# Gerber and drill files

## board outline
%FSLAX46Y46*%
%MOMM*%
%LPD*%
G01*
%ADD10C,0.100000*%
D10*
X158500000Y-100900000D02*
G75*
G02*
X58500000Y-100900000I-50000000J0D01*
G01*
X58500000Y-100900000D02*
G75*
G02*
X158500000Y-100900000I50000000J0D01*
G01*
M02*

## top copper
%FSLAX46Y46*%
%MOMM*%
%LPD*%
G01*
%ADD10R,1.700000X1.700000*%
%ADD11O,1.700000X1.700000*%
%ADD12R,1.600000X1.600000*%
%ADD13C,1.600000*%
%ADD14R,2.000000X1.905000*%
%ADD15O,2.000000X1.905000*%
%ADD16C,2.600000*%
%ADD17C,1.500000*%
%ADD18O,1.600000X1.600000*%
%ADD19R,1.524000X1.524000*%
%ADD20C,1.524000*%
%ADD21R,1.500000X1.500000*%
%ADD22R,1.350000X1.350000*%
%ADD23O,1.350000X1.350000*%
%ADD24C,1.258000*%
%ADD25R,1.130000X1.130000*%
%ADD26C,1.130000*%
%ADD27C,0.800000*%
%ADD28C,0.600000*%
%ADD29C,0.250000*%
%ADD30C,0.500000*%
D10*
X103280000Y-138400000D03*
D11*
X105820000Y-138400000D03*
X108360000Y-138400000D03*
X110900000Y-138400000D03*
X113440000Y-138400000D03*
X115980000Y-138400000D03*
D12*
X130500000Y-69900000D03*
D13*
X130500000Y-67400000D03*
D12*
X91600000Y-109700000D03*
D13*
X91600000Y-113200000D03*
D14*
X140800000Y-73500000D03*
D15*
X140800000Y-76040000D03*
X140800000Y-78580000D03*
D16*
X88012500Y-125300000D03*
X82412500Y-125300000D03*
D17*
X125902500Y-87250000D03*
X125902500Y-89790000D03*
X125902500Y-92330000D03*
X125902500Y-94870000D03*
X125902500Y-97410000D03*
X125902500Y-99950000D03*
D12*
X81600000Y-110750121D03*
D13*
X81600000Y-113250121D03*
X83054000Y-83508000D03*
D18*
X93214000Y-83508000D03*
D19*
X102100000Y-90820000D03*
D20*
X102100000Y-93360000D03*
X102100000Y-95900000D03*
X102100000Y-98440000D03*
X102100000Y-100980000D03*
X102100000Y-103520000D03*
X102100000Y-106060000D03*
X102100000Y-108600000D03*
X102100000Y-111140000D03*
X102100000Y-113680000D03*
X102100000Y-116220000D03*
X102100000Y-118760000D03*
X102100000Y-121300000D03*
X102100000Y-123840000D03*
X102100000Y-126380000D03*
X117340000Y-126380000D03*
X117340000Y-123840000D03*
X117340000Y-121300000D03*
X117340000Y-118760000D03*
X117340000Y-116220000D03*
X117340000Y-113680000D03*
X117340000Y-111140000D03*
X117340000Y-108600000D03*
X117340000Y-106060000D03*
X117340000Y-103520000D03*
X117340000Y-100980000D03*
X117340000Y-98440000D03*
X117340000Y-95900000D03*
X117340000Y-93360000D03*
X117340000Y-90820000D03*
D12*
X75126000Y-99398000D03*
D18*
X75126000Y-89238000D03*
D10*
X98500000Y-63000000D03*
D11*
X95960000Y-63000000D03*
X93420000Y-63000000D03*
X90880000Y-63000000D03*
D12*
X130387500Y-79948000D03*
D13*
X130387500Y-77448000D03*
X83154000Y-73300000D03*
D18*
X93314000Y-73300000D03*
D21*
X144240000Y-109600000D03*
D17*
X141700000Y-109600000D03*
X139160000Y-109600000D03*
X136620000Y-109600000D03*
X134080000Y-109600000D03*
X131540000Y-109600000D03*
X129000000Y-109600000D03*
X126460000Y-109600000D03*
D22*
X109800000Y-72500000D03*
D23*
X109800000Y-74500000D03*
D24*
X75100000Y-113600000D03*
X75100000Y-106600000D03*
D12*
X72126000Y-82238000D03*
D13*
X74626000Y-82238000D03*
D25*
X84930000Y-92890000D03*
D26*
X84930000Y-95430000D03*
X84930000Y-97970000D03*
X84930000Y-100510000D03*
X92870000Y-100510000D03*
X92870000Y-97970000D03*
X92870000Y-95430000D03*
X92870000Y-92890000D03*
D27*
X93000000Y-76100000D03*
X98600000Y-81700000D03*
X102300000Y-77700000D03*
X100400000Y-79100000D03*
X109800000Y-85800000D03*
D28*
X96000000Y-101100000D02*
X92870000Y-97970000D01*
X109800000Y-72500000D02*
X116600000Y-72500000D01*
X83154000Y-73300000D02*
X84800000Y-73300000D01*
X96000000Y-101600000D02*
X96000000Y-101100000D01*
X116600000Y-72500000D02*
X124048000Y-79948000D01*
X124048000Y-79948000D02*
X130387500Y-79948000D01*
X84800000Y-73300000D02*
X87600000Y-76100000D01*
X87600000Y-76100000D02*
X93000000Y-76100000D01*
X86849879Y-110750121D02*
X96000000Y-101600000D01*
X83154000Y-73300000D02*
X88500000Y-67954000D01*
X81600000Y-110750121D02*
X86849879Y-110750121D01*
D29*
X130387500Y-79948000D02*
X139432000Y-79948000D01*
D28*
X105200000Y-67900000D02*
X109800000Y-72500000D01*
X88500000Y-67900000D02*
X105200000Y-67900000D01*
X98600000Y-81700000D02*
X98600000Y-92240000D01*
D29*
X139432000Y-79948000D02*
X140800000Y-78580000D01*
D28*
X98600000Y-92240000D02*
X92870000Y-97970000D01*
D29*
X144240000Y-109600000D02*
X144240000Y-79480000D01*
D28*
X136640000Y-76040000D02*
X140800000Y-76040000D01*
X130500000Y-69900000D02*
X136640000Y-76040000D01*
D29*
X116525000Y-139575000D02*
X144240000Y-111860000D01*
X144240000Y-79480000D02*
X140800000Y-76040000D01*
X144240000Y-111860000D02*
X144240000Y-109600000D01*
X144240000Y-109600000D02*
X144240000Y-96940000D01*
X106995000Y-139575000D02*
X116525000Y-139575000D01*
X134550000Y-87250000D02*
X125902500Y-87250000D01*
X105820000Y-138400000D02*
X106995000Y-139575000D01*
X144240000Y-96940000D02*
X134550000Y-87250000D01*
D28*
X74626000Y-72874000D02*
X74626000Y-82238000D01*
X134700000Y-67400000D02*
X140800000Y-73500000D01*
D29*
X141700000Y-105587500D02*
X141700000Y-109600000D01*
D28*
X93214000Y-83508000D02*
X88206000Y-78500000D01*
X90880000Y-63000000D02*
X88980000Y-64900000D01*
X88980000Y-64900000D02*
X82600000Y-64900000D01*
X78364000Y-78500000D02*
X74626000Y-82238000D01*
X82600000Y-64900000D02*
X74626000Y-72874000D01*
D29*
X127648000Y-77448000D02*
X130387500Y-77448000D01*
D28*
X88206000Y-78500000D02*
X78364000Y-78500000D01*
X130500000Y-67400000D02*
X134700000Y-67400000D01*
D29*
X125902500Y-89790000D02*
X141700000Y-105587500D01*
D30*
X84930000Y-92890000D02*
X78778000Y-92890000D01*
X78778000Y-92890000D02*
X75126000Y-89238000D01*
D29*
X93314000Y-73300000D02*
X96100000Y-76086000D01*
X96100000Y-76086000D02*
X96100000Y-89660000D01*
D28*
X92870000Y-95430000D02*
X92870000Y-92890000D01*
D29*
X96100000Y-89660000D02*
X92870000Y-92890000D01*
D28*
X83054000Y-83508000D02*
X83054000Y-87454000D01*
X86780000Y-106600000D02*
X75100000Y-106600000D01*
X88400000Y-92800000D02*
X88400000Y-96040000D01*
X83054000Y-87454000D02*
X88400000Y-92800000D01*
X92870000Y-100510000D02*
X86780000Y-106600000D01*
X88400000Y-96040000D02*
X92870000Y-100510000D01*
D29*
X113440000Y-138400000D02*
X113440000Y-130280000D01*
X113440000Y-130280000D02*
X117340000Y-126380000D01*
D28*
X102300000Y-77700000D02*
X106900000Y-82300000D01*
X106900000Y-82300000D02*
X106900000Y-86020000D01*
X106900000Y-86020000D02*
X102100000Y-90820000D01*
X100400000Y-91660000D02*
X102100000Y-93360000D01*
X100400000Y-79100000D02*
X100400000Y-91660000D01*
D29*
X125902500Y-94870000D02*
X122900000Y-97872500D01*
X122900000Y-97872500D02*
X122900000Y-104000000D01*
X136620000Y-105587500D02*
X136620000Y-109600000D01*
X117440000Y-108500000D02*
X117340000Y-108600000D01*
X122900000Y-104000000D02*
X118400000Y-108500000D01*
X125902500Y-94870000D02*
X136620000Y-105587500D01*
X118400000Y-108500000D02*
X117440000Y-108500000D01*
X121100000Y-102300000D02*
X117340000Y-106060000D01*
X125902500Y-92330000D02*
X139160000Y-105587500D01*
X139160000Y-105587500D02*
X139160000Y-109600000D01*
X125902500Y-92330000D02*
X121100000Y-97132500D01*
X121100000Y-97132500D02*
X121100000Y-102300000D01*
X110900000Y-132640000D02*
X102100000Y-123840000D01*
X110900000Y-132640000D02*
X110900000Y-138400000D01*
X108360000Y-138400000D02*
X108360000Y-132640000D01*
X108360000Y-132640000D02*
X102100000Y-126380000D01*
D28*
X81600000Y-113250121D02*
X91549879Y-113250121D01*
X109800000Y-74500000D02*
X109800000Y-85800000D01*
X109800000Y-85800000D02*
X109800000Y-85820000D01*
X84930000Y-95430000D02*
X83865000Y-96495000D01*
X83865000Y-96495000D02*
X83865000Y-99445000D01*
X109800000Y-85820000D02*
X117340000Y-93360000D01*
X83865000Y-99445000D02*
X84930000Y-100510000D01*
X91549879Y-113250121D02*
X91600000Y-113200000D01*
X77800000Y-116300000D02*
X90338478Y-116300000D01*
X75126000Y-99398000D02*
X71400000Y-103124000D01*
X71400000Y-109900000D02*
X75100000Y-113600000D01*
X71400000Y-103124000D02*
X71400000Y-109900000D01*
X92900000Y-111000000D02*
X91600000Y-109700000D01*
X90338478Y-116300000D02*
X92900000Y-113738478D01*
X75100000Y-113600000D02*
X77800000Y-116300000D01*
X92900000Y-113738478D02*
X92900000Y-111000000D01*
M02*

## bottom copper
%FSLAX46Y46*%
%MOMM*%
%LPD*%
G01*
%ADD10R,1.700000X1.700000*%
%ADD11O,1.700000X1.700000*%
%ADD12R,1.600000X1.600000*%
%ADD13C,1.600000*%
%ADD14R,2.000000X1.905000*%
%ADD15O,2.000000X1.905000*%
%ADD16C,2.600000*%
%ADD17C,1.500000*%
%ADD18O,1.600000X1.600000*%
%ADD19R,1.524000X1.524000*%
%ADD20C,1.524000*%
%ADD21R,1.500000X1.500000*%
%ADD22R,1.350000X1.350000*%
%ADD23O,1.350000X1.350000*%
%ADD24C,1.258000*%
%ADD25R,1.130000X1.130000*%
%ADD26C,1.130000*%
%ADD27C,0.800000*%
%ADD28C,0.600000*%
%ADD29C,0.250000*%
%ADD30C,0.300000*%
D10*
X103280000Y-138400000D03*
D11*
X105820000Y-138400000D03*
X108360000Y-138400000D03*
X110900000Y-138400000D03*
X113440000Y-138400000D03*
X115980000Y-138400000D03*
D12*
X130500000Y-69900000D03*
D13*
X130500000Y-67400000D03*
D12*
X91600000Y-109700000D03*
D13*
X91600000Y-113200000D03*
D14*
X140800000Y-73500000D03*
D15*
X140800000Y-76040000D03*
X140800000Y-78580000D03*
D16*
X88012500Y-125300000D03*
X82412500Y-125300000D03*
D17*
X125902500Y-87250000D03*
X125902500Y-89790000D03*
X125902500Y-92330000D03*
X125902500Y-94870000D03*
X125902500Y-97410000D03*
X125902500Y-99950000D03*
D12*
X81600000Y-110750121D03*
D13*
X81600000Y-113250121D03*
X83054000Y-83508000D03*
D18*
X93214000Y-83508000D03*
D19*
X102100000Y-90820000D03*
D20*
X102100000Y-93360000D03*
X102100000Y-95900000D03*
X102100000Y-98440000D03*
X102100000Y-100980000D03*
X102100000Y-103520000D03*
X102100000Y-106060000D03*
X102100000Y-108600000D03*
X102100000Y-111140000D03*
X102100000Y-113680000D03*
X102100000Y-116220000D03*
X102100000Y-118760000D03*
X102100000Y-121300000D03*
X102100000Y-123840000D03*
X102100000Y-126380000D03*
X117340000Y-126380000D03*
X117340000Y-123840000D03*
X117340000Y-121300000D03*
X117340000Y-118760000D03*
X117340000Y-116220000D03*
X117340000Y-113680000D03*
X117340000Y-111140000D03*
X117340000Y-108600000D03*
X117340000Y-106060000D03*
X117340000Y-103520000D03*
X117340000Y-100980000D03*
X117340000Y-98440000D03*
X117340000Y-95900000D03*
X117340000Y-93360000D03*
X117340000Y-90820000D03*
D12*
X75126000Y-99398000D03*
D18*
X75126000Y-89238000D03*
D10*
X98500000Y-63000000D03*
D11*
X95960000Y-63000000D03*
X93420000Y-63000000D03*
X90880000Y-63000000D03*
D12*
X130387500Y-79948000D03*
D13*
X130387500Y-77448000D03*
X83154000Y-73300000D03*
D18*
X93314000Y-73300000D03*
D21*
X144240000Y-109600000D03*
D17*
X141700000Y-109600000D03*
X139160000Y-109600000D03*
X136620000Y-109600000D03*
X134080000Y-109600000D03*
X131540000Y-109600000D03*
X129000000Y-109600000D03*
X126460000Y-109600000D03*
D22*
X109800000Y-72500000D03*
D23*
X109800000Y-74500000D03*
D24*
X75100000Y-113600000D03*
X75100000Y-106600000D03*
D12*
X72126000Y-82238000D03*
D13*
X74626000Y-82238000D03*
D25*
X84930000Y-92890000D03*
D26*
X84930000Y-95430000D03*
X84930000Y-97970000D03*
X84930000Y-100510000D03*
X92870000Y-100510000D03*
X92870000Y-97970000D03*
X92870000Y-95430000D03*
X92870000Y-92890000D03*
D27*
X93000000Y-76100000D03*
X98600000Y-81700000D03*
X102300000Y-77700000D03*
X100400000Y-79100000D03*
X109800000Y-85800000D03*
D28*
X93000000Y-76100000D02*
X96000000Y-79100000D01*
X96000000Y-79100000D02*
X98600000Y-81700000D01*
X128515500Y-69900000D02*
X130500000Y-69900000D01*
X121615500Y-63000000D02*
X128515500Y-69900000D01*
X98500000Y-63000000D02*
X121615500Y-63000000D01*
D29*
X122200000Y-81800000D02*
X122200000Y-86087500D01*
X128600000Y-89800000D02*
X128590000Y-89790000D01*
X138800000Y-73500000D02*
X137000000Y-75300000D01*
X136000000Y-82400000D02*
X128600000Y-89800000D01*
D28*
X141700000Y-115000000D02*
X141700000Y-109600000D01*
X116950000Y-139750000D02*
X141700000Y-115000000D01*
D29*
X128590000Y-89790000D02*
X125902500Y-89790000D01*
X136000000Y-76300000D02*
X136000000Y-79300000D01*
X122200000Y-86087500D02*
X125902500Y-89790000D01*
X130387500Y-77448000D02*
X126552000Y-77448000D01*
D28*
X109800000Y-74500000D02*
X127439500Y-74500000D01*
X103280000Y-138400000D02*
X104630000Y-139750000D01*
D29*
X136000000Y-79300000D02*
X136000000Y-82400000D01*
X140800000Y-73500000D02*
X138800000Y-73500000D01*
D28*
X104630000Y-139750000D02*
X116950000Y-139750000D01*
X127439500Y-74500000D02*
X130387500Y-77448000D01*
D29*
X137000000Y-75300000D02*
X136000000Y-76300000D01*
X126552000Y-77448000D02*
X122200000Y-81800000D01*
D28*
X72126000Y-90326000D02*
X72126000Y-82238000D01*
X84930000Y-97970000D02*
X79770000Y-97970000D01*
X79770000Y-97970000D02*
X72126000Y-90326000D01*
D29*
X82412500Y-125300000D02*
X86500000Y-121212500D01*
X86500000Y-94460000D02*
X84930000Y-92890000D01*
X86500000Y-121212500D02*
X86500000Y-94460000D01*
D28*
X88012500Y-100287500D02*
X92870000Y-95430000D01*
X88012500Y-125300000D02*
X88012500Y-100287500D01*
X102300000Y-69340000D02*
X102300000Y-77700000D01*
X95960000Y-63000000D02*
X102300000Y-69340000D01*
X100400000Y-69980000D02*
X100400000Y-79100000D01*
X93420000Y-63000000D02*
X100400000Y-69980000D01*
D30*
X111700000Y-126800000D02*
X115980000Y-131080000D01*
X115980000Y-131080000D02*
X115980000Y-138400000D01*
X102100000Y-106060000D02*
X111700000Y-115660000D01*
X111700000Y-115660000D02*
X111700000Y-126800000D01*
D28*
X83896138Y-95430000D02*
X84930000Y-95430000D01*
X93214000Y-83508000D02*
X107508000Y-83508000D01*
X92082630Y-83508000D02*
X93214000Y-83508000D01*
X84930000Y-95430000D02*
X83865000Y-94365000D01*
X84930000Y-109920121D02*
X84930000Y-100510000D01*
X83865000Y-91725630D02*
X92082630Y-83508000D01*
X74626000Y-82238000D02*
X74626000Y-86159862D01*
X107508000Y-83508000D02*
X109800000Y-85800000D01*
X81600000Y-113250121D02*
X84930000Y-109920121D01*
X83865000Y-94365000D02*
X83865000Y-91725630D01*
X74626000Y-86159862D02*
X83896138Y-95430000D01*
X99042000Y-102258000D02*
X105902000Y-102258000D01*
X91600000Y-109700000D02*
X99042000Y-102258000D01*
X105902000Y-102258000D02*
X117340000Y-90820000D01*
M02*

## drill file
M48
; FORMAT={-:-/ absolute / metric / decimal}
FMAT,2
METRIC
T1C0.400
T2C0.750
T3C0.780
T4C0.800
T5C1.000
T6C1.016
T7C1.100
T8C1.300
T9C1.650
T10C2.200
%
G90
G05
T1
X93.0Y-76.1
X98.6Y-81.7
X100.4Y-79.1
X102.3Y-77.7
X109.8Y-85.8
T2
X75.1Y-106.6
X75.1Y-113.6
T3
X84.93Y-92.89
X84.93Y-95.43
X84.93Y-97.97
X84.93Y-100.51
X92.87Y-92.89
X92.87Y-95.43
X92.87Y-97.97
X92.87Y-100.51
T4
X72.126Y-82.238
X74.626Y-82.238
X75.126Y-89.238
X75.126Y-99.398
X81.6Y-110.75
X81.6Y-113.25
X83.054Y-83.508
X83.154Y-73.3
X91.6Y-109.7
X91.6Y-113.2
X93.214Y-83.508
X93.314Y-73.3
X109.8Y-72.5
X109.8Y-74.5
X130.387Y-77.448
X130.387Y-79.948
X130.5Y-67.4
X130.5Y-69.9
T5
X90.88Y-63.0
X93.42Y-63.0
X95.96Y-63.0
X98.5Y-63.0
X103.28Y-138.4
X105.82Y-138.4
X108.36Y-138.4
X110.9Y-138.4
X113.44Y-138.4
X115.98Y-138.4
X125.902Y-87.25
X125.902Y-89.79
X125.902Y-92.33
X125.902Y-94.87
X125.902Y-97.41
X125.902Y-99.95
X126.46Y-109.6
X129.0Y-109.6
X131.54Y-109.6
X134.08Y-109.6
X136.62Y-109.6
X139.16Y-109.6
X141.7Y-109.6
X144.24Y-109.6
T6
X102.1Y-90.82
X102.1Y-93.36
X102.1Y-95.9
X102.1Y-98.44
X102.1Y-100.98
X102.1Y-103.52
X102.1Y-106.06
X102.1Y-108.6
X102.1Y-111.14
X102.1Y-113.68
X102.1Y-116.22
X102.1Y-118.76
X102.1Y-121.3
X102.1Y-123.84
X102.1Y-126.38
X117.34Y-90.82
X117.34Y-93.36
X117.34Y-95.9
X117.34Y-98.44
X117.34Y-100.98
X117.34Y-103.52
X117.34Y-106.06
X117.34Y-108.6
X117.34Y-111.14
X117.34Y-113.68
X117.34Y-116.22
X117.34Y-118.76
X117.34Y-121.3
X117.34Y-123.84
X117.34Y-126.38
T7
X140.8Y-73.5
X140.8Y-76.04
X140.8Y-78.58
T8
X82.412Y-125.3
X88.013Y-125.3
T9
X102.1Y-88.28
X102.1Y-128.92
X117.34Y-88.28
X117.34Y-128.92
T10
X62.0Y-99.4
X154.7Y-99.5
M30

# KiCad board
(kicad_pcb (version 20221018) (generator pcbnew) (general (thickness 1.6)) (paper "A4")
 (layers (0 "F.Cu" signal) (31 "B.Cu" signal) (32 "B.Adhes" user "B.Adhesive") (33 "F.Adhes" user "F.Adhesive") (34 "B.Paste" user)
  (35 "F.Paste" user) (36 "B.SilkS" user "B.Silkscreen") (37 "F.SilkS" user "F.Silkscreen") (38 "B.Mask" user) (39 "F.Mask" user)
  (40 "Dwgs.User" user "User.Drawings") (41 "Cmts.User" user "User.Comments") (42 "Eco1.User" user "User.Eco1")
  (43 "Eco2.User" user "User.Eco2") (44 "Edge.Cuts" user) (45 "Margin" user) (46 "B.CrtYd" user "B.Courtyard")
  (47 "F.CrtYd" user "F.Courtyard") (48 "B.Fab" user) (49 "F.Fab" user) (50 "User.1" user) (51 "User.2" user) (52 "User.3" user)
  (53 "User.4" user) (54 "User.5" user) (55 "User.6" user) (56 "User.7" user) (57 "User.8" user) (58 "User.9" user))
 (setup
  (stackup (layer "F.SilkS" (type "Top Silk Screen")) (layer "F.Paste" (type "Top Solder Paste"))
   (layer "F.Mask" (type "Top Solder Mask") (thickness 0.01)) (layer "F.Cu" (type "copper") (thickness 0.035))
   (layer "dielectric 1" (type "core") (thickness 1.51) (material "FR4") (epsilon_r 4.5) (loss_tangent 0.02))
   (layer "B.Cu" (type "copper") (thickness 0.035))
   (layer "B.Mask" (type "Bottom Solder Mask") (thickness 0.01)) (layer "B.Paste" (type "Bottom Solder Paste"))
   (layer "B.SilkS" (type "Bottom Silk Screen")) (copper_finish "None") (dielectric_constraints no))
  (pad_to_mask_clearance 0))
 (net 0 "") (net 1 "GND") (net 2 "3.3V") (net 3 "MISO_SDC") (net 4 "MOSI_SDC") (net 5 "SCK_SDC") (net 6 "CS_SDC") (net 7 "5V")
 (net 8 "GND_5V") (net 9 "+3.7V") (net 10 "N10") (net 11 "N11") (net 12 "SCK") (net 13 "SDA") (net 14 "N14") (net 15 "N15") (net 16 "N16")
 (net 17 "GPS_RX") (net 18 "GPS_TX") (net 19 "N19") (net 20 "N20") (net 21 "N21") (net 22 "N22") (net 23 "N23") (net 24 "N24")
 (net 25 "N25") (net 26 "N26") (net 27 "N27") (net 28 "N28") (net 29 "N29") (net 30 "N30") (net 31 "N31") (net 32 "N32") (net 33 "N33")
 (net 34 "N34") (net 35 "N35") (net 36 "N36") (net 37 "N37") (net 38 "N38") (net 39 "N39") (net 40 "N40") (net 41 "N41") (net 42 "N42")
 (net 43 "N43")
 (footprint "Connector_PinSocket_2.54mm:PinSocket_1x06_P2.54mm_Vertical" (layer "F.Cu") (at 103.28 138.4 90)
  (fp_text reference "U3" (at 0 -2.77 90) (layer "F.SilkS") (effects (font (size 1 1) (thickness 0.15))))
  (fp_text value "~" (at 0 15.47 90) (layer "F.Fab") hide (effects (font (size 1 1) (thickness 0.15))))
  (pad "1" thru_hole rect (at 0 0 90) (size 1.7 1.7) (drill 1) (layers "*.Cu" "*.Mask") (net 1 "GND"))
  (pad "2" thru_hole oval (at 0 2.54 90) (size 1.7 1.7) (drill 1) (layers "*.Cu" "*.Mask") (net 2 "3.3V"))
  (pad "3" thru_hole oval (at 0 5.08 90) (size 1.7 1.7) (drill 1) (layers "*.Cu" "*.Mask") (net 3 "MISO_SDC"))
  (pad "4" thru_hole oval (at 0 7.62 90) (size 1.7 1.7) (drill 1) (layers "*.Cu" "*.Mask") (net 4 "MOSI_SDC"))
  (pad "5" thru_hole oval (at 0 10.16 90) (size 1.7 1.7) (drill 1) (layers "*.Cu" "*.Mask") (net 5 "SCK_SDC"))
  (pad "6" thru_hole oval (at 0 12.7 90) (size 1.7 1.7) (drill 1) (layers "*.Cu" "*.Mask") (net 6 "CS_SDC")))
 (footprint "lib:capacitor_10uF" (layer "F.Cu") (at 135.5 67.9 90)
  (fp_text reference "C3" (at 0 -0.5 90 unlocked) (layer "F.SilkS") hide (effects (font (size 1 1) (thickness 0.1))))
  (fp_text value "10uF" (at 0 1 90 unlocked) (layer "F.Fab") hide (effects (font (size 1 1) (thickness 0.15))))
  (pad "1" thru_hole rect (at -2 -5 90) (size 1.6 1.6) (drill 0.8) (layers "*.Cu" "*.Mask") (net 2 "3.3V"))
  (pad "2" thru_hole circle (at 0.5 -5 90) (size 1.6 1.6) (drill 0.8) (layers "*.Cu" "*.Mask") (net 1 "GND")))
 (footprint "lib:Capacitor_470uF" (layer "F.Cu") (at 91.56 111.051 -90)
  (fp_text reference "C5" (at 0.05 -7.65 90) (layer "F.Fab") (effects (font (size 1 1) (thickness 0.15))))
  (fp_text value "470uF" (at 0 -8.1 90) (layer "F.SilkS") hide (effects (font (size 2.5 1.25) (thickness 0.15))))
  (pad "1" thru_hole rect (at -1.351 -0.04 270) (size 1.6 1.6) (drill 0.8) (layers "*.Cu" "*.Mask") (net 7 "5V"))
  (pad "2" thru_hole circle (at 2.149 -0.04 270) (size 1.6 1.6) (drill 0.8) (layers "*.Cu" "*.Mask") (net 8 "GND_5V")))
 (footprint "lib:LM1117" (layer "F.Cu") (at 145 76.09 -90)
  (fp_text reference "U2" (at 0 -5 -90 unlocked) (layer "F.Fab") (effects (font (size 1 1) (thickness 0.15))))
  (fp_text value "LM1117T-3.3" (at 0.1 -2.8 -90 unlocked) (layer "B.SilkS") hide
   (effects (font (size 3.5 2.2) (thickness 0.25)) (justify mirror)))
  (pad "1" thru_hole rect (at -2.59 4.2 270) (size 1.905 2) (drill 1.1) (layers "*.Cu" "*.Mask") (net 1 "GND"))
  (pad "2" thru_hole oval (at -0.05 4.2 270) (size 1.905 2) (drill 1.1) (layers "*.Cu" "*.Mask") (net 2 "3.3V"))
  (pad "3" thru_hole oval (at 2.49 4.2 270) (size 1.905 2) (drill 1.1) (layers "*.Cu" "*.Mask") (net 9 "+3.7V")))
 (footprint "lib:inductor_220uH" (layer "F.Cu") (at 78.0125 124.3 -90)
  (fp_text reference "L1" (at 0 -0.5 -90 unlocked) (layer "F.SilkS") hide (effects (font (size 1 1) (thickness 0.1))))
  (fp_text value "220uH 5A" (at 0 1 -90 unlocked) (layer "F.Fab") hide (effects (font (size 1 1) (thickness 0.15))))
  (pad "1" thru_hole circle (at 1 -10 270) (size 2.6 2.6) (drill 1.3) (layers "*.Cu" "*.Mask") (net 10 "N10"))
  (pad "2" thru_hole circle (at 1 -4.4 270) (size 2.6 2.6) (drill 1.3) (layers "*.Cu" "*.Mask") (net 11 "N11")))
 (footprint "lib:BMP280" (layer "F.Cu") (at 131.37 93.45 -90)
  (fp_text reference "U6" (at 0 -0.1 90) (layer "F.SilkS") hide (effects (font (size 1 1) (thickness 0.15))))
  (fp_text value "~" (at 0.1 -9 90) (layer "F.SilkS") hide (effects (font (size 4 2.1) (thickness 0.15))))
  (pad "1" thru_hole circle (at -6.2 5.4675 270) (size 1.5 1.5) (drill 1) (layers "*.Cu" "*.Mask") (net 2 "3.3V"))
  (pad "2" thru_hole circle (at -3.66 5.4675 270) (size 1.5 1.5) (drill 1) (layers "*.Cu" "*.Mask") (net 1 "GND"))
  (pad "3" thru_hole circle (at -1.12 5.4675 270) (size 1.5 1.5) (drill 1) (layers "*.Cu" "*.Mask") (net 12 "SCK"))
  (pad "4" thru_hole circle (at 1.42 5.4675 270) (size 1.5 1.5) (drill 1) (layers "*.Cu" "*.Mask") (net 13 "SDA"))
  (pad "5" thru_hole circle (at 3.96 5.4675 270) (size 1.5 1.5) (drill 1) (layers "*.Cu" "*.Mask") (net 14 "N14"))
  (pad "6" thru_hole circle (at 6.5 5.4675 270) (size 1.5 1.5) (drill 1) (layers "*.Cu" "*.Mask") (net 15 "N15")))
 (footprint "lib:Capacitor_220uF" (layer "F.Cu") (at 81.339 111.34988 -90)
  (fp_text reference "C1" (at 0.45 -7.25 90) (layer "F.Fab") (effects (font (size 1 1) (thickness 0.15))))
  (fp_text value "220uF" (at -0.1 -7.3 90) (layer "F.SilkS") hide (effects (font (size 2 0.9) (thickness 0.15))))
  (pad "1" thru_hole rect (at -0.599759 -0.261 270) (size 1.6 1.6) (drill 0.8) (layers "*.Cu" "*.Mask") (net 9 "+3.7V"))
  (pad "2" thru_hole circle (at 1.900241 -0.261 270) (size 1.6 1.6) (drill 0.8) (layers "*.Cu" "*.Mask") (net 8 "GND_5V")))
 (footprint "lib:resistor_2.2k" (layer "F.Cu") (at 88.1 81.5)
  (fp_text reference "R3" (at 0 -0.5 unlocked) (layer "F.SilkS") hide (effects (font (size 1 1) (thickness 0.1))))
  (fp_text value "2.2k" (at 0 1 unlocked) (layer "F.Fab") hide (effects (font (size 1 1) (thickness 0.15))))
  (pad "1" thru_hole circle (at -5.046 2.008) (size 1.6 1.6) (drill 0.8) (layers "*.Cu" "*.Mask") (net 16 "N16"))
  (pad "2" thru_hole oval (at 5.114 2.008) (size 1.6 1.6) (drill 0.8) (layers "*.Cu" "*.Mask") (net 8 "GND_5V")))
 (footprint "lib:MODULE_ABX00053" (layer "F.Cu") (at 109.72 108.6 -90)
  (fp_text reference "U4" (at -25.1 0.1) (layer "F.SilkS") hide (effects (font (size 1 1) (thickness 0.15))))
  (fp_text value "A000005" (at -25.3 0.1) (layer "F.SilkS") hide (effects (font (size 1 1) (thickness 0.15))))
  (pad "" np_thru_hole circle (at -20.32 -7.62 270) (size 1.65 1.65) (drill 1.65) (layers "*.Cu" "*.Mask"))
  (pad "" np_thru_hole circle (at -20.32 7.62 270) (size 1.65 1.65) (drill 1.65) (layers "*.Cu" "*.Mask"))
  (pad "" np_thru_hole circle (at 20.32 -7.62 270) (size 1.65 1.65) (drill 1.65) (layers "*.Cu" "*.Mask"))
  (pad "" np_thru_hole circle (at 20.32 7.62 270) (size 1.65 1.65) (drill 1.65) (layers "*.Cu" "*.Mask"))
  (pad "1" thru_hole rect (at -17.78 7.62 270) (size 1.524 1.524) (drill 1.016) (layers "*.Cu" "*.Mask") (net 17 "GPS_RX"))
  (pad "2" thru_hole circle (at -15.24 7.62 270) (size 1.524 1.524) (drill 1.016) (layers "*.Cu" "*.Mask") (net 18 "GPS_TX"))
  (pad "3" thru_hole circle (at -12.7 7.62 270) (size 1.524 1.524) (drill 1.016) (layers "*.Cu" "*.Mask") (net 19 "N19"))
  (pad "4" thru_hole circle (at -10.16 7.62 270) (size 1.524 1.524) (drill 1.016) (layers "*.Cu" "*.Mask") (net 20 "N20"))
  (pad "5" thru_hole circle (at -7.62 7.62 270) (size 1.524 1.524) (drill 1.016) (layers "*.Cu" "*.Mask") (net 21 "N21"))
  (pad "6" thru_hole circle (at -5.08 7.62 270) (size 1.524 1.524) (drill 1.016) (layers "*.Cu" "*.Mask") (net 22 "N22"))
  (pad "7" thru_hole circle (at -2.54 7.62 270) (size 1.524 1.524) (drill 1.016) (layers "*.Cu" "*.Mask") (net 6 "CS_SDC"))
  (pad "8" thru_hole circle (at 0 7.62 270) (size 1.524 1.524) (drill 1.016) (layers "*.Cu" "*.Mask") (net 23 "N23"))
  (pad "9" thru_hole circle (at 2.54 7.62 270) (size 1.524 1.524) (drill 1.016) (layers "*.Cu" "*.Mask") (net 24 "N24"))
  (pad "10" thru_hole circle (at 5.08 7.62 270) (size 1.524 1.524) (drill 1.016) (layers "*.Cu" "*.Mask") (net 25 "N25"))
  (pad "11" thru_hole circle (at 7.62 7.62 270) (size 1.524 1.524) (drill 1.016) (layers "*.Cu" "*.Mask") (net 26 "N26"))
  (pad "12" thru_hole circle (at 10.16 7.62 270) (size 1.524 1.524) (drill 1.016) (layers "*.Cu" "*.Mask") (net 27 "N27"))
  (pad "13" thru_hole circle (at 12.7 7.62 270) (size 1.524 1.524) (drill 1.016) (layers "*.Cu" "*.Mask") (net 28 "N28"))
  (pad "14" thru_hole circle (at 15.24 7.62 270) (size 1.524 1.524) (drill 1.016) (layers "*.Cu" "*.Mask") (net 4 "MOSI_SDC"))
  (pad "15" thru_hole circle (at 17.78 7.62 270) (size 1.524 1.524) (drill 1.016) (layers "*.Cu" "*.Mask") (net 3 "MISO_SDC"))
  (pad "16" thru_hole circle (at 17.78 -7.62 270) (size 1.524 1.524) (drill 1.016) (layers "*.Cu" "*.Mask") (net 5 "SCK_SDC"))
  (pad "17" thru_hole circle (at 15.24 -7.62 270) (size 1.524 1.524) (drill 1.016) (layers "*.Cu" "*.Mask") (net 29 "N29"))
  (pad "18" thru_hole circle (at 12.7 -7.62 270) (size 1.524 1.524) (drill 1.016) (layers "*.Cu" "*.Mask") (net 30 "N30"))
  (pad "19" thru_hole circle (at 10.16 -7.62 270) (size 1.524 1.524) (drill 1.016) (layers "*.Cu" "*.Mask") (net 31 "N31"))
  (pad "20" thru_hole circle (at 7.62 -7.62 270) (size 1.524 1.524) (drill 1.016) (layers "*.Cu" "*.Mask") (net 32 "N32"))
  (pad "21" thru_hole circle (at 5.08 -7.62 270) (size 1.524 1.524) (drill 1.016) (layers "*.Cu" "*.Mask") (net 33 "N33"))
  (pad "22" thru_hole circle (at 2.54 -7.62 270) (size 1.524 1.524) (drill 1.016) (layers "*.Cu" "*.Mask") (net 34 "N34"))
  (pad "23" thru_hole circle (at 0 -7.62 270) (size 1.524 1.524) (drill 1.016) (layers "*.Cu" "*.Mask") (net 13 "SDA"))
  (pad "24" thru_hole circle (at -2.54 -7.62 270) (size 1.524 1.524) (drill 1.016) (layers "*.Cu" "*.Mask") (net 12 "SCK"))
  (pad "25" thru_hole circle (at -5.08 -7.62 270) (size 1.524 1.524) (drill 1.016) (layers "*.Cu" "*.Mask") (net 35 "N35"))
  (pad "26" thru_hole circle (at -7.62 -7.62 270) (size 1.524 1.524) (drill 1.016) (layers "*.Cu" "*.Mask") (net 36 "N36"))
  (pad "27" thru_hole circle (at -10.16 -7.62 270) (size 1.524 1.524) (drill 1.016) (layers "*.Cu" "*.Mask") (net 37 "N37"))
  (pad "28" thru_hole circle (at -12.7 -7.62 270) (size 1.524 1.524) (drill 1.016) (layers "*.Cu" "*.Mask") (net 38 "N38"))
  (pad "29" thru_hole circle (at -15.24 -7.62 270) (size 1.524 1.524) (drill 1.016) (layers "*.Cu" "*.Mask") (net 8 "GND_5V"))
  (pad "30" thru_hole circle (at -17.78 -7.62 270) (size 1.524 1.524) (drill 1.016) (layers "*.Cu" "*.Mask") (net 7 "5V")))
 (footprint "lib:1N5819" (layer "F.Cu") (at 78.476 93.748 90)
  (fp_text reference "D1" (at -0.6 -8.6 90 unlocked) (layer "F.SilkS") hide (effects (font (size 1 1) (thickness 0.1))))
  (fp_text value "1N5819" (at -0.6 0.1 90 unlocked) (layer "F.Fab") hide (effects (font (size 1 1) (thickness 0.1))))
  (pad "1" thru_hole rect (at -5.65 -3.35 90) (size 1.6 1.6) (drill 0.8) (layers "*.Cu" "*.Mask") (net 7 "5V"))
  (pad "2" thru_hole oval (at 4.51 -3.35 90) (size 1.6 1.6) (drill 0.8) (layers "*.Cu" "*.Mask") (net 11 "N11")))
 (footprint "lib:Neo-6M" (layer "F.Cu") (at 95.16 67)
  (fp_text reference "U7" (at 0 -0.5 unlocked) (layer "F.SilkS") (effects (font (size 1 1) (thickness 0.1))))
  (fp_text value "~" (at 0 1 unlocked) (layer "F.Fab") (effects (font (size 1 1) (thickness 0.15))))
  (pad "1" thru_hole rect (at 3.34 -4 270) (size 1.7 1.7) (drill 1) (layers "*.Cu" "*.Mask") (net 2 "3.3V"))
  (pad "2" thru_hole oval (at 0.8 -4 270) (size 1.7 1.7) (drill 1) (layers "*.Cu" "*.Mask") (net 17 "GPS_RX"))
  (pad "3" thru_hole oval (at -1.74 -4 270) (size 1.7 1.7) (drill 1) (layers "*.Cu" "*.Mask") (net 18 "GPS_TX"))
  (pad "4" thru_hole oval (at -4.28 -4 270) (size 1.7 1.7) (drill 1) (layers "*.Cu" "*.Mask") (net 1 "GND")))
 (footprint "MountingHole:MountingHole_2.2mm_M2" (layer "F.Cu") (at 62 99.4)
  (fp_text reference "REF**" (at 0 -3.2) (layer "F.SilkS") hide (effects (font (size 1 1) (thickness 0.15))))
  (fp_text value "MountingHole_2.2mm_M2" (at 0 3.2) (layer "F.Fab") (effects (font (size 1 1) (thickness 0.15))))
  (pad "" np_thru_hole circle (at 0 0) (size 2.2 2.2) (drill 2.2) (layers "*.Cu" "*.Mask")))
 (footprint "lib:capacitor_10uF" (layer "F.Cu") (at 135.3875 77.948 90)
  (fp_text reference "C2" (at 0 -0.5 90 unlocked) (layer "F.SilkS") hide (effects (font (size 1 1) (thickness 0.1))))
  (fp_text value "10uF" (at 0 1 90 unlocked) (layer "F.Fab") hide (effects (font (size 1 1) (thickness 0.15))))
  (pad "1" thru_hole rect (at -2 -5 90) (size 1.6 1.6) (drill 0.8) (layers "*.Cu" "*.Mask") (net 9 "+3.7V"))
  (pad "2" thru_hole circle (at 0.5 -5 90) (size 1.6 1.6) (drill 0.8) (layers "*.Cu" "*.Mask") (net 1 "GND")))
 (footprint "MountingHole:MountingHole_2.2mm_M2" (layer "F.Cu") (at 154.7 99.5)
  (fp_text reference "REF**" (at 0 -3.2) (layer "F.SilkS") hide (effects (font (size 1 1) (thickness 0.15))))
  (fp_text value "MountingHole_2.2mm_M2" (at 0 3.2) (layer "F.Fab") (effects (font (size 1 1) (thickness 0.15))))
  (pad "" np_thru_hole circle (at 0 0) (size 2.2 2.2) (drill 2.2) (layers "*.Cu" "*.Mask")))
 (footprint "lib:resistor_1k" (layer "F.Cu") (at 88.2 71.8)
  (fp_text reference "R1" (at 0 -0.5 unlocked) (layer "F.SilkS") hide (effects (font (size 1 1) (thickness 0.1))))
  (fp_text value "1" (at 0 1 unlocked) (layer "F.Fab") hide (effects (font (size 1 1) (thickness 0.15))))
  (pad "1" thru_hole circle (at -5.046 1.5) (size 1.6 1.6) (drill 0.8) (layers "*.Cu" "*.Mask") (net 9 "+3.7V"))
  (pad "2" thru_hole oval (at 5.114 1.5) (size 1.6 1.6) (drill 0.8) (layers "*.Cu" "*.Mask") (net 10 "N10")))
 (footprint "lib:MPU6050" (layer "F.Cu") (at 134.08 101.98 180)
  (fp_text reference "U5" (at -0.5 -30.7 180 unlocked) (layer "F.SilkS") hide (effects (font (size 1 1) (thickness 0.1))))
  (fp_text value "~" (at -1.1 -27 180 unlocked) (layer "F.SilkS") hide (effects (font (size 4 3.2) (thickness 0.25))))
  (pad "1" thru_hole rect (at -10.16 -7.62 180) (size 1.5 1.5) (drill 1) (layers "*.Cu" "*.Mask") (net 2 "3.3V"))
  (pad "2" thru_hole circle (at -7.62 -7.62 180) (size 1.5 1.5) (drill 1) (layers "*.Cu" "*.Mask") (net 1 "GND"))
  (pad "3" thru_hole circle (at -5.08 -7.62 180) (size 1.5 1.5) (drill 1) (layers "*.Cu" "*.Mask") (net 12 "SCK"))
  (pad "4" thru_hole circle (at -2.54 -7.62 180) (size 1.5 1.5) (drill 1) (layers "*.Cu" "*.Mask") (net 13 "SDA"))
  (pad "5" thru_hole circle (at 0 -7.62 180) (size 1.5 1.5) (drill 1) (layers "*.Cu" "*.Mask") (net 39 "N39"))
  (pad "6" thru_hole circle (at 2.54 -7.62 180) (size 1.5 1.5) (drill 1) (layers "*.Cu" "*.Mask") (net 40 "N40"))
  (pad "7" thru_hole circle (at 5.08 -7.62 180) (size 1.5 1.5) (drill 1) (layers "*.Cu" "*.Mask") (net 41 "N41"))
  (pad "8" thru_hole circle (at 7.62 -7.62 180) (size 1.5 1.5) (drill 1) (layers "*.Cu" "*.Mask") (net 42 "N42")))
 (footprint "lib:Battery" (layer "F.Cu") (at 110.302 78.816)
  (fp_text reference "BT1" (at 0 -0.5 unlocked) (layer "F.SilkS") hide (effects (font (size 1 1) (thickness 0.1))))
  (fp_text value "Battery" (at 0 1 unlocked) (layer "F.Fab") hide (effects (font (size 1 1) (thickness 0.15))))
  (pad "1" thru_hole rect (at -0.502 -6.316) (size 1.35 1.35) (drill 0.8) (layers "*.Cu" "*.Mask") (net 9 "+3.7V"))
  (pad "2" thru_hole oval (at -0.502 -4.316) (size 1.35 1.35) (drill 0.8) (layers "*.Cu" "*.Mask") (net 8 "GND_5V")))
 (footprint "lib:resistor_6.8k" (layer "F.Cu") (at 75.1 110.1 90)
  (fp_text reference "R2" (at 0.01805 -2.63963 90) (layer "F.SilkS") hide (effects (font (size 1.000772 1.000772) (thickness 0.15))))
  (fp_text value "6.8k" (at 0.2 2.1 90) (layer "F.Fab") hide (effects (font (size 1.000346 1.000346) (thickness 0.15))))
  (pad "1" thru_hole circle (at -3.5 0 90) (size 1.258 1.258) (drill 0.75) (layers "*.Cu" "*.Mask") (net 7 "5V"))
  (pad "2" thru_hole circle (at 3.5 0 90) (size 1.258 1.258) (drill 0.75) (layers "*.Cu" "*.Mask") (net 16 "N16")))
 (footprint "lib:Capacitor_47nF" (layer "F.Cu") (at 73.126 80.238)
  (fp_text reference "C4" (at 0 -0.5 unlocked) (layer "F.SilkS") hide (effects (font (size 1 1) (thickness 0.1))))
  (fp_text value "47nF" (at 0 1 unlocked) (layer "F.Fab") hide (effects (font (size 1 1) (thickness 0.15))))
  (pad "1" thru_hole rect (at -1 2) (size 1.6 1.6) (drill 0.8) (layers "*.Cu" "*.Mask") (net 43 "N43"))
  (pad "2" thru_hole circle (at 1.5 2) (size 1.6 1.6) (drill 0.8) (layers "*.Cu" "*.Mask") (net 8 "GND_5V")))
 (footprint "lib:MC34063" (layer "F.Cu") (at 88.9 96.7)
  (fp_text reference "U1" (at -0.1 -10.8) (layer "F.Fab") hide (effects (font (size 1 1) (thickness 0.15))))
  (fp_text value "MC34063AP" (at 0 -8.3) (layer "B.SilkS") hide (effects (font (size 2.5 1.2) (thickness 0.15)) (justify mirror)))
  (pad "1" thru_hole rect (at -3.97 -3.81) (size 1.13 1.13) (drill 0.78) (layers "*.Cu" "*.Mask") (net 11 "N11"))
  (pad "2" thru_hole circle (at -3.97 -1.27) (size 1.13 1.13) (drill 0.78) (layers "*.Cu" "*.Mask") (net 8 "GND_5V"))
  (pad "3" thru_hole circle (at -3.97 1.27) (size 1.13 1.13) (drill 0.78) (layers "*.Cu" "*.Mask") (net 43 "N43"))
  (pad "4" thru_hole circle (at -3.97 3.81) (size 1.13 1.13) (drill 0.78) (layers "*.Cu" "*.Mask") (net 8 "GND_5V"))
  (pad "5" thru_hole circle (at 3.97 3.81) (size 1.13 1.13) (drill 0.78) (layers "*.Cu" "*.Mask") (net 16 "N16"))
  (pad "6" thru_hole circle (at 3.97 1.27) (size 1.13 1.13) (drill 0.78) (layers "*.Cu" "*.Mask") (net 9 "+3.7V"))
  (pad "7" thru_hole circle (at 3.97 -1.27) (size 1.13 1.13) (drill 0.78) (layers "*.Cu" "*.Mask") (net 10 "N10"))
  (pad "8" thru_hole circle (at 3.97 -3.81) (size 1.13 1.13) (drill 0.78) (layers "*.Cu" "*.Mask") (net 10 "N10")))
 (gr_circle (center 108.5 100.9) (end 158.5 100.9) (stroke (width 0.1) (type default)) (fill none) (layer "Edge.Cuts"))
 (segment (start 96 101.1) (end 92.87 97.97) (width 0.6) (layer "F.Cu") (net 9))
 (segment (start 109.8 72.5) (end 116.6 72.5) (width 0.6) (layer "F.Cu") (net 9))
 (segment (start 83.154 73.3) (end 84.8 73.3) (width 0.6) (layer "F.Cu") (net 9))
 (segment (start 96 101.6) (end 96 101.1) (width 0.6) (layer "F.Cu") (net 9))
 (segment (start 116.6 72.5) (end 124.048 79.948) (width 0.6) (layer "F.Cu") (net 9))
 (segment (start 124.048 79.948) (end 130.3875 79.948) (width 0.6) (layer "F.Cu") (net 9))
 (segment (start 84.8 73.3) (end 87.6 76.1) (width 0.6) (layer "F.Cu") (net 9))
 (segment (start 87.6 76.1) (end 93 76.1) (width 0.6) (layer "F.Cu") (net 9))
 (segment (start 86.849879 110.750121) (end 96 101.6) (width 0.6) (layer "F.Cu") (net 9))
 (segment (start 83.154 73.3) (end 88.5 67.954) (width 0.6) (layer "F.Cu") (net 9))
 (segment (start 81.6 110.750121) (end 86.849879 110.750121) (width 0.6) (layer "F.Cu") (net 9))
 (segment (start 130.3875 79.948) (end 139.432 79.948) (width 0.25) (layer "F.Cu") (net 9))
 (segment (start 105.2 67.9) (end 109.8 72.5) (width 0.6) (layer "F.Cu") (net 9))
 (segment (start 88.5 67.9) (end 105.2 67.9) (width 0.6) (layer "F.Cu") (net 9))
 (segment (start 98.6 81.7) (end 98.6 92.24) (width 0.6) (layer "F.Cu") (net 9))
 (segment (start 139.432 79.948) (end 140.8 78.58) (width 0.25) (layer "F.Cu") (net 9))
 (segment (start 98.6 92.24) (end 92.87 97.97) (width 0.6) (layer "F.Cu") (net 9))
 (via (at 93 76.1) (size 0.8) (drill 0.4) (layers "F.Cu" "B.Cu") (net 9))
 (via (at 98.6 81.7) (size 0.8) (drill 0.4) (layers "F.Cu" "B.Cu") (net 9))
 (segment (start 93 76.1) (end 96 79.1) (width 0.6) (layer "B.Cu") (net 9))
 (segment (start 96 79.1) (end 98.6 81.7) (width 0.6) (layer "B.Cu") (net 9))
 (segment (start 144.24 109.6) (end 144.24 79.48) (width 0.25) (layer "F.Cu") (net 2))
 (segment (start 136.64 76.04) (end 140.8 76.04) (width 0.6) (layer "F.Cu") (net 2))
 (segment (start 130.5 69.9) (end 136.64 76.04) (width 0.6) (layer "F.Cu") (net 2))
 (segment (start 116.525 139.575) (end 144.24 111.86) (width 0.25) (layer "F.Cu") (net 2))
 (segment (start 144.24 79.48) (end 140.8 76.04) (width 0.25) (layer "F.Cu") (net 2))
 (segment (start 144.24 111.86) (end 144.24 109.6) (width 0.25) (layer "F.Cu") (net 2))
 (segment (start 144.24 109.6) (end 144.24 96.94) (width 0.25) (layer "F.Cu") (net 2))
 (segment (start 106.995 139.575) (end 116.525 139.575) (width 0.25) (layer "F.Cu") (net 2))
 (segment (start 134.55 87.25) (end 125.9025 87.25) (width 0.25) (layer "F.Cu") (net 2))
 (segment (start 105.82 138.4) (end 106.995 139.575) (width 0.25) (layer "F.Cu") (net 2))
 (segment (start 144.24 96.94) (end 134.55 87.25) (width 0.25) (layer "F.Cu") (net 2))
 (segment (start 128.5155 69.9) (end 130.5 69.9) (width 0.6) (layer "B.Cu") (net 2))
 (segment (start 121.6155 63) (end 128.5155 69.9) (width 0.6) (layer "B.Cu") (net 2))
 (segment (start 98.5 63) (end 121.6155 63) (width 0.6) (layer "B.Cu") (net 2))
 (segment (start 74.626 72.874) (end 74.626 82.238) (width 0.6) (layer "F.Cu") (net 1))
 (segment (start 134.7 67.4) (end 140.8 73.5) (width 0.6) (layer "F.Cu") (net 1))
 (segment (start 141.7 105.5875) (end 141.7 109.6) (width 0.25) (layer "F.Cu") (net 1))
 (segment (start 93.214 83.508) (end 88.206 78.5) (width 0.6) (layer "F.Cu") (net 1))
 (segment (start 90.88 63) (end 88.98 64.9) (width 0.6) (layer "F.Cu") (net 1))
 (segment (start 88.98 64.9) (end 82.6 64.9) (width 0.6) (layer "F.Cu") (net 1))
 (segment (start 78.364 78.5) (end 74.626 82.238) (width 0.6) (layer "F.Cu") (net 1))
 (segment (start 82.6 64.9) (end 74.626 72.874) (width 0.6) (layer "F.Cu") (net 1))
 (segment (start 127.648 77.448) (end 130.3875 77.448) (width 0.25) (layer "F.Cu") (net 1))
 (segment (start 88.206 78.5) (end 78.364 78.5) (width 0.6) (layer "F.Cu") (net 1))
 (segment (start 130.5 67.4) (end 134.7 67.4) (width 0.6) (layer "F.Cu") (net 1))
 (segment (start 125.9025 89.79) (end 141.7 105.5875) (width 0.25) (layer "F.Cu") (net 1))
 (segment (start 122.2 81.8) (end 122.2 86.0875) (width 0.25) (layer "B.Cu") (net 1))
 (segment (start 128.6 89.8) (end 128.59 89.79) (width 0.25) (layer "B.Cu") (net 1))
 (segment (start 138.8 73.5) (end 137 75.3) (width 0.25) (layer "B.Cu") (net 1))
 (segment (start 136 82.4) (end 128.6 89.8) (width 0.25) (layer "B.Cu") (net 1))
 (segment (start 141.7 115) (end 141.7 109.6) (width 0.6) (layer "B.Cu") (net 1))
 (segment (start 116.95 139.75) (end 141.7 115) (width 0.6) (layer "B.Cu") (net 1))
 (segment (start 128.59 89.79) (end 125.9025 89.79) (width 0.25) (layer "B.Cu") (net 1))
 (segment (start 136 76.3) (end 136 79.3) (width 0.25) (layer "B.Cu") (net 1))
 (segment (start 122.2 86.0875) (end 125.9025 89.79) (width 0.25) (layer "B.Cu") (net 1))
 (segment (start 130.3875 77.448) (end 126.552 77.448) (width 0.25) (layer "B.Cu") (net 1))
 (segment (start 109.8 74.5) (end 127.4395 74.5) (width 0.6) (layer "B.Cu") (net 1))
 (segment (start 103.28 138.4) (end 104.63 139.75) (width 0.6) (layer "B.Cu") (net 1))
 (segment (start 136 79.3) (end 136 82.4) (width 0.25) (layer "B.Cu") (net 1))
 (segment (start 140.8 73.5) (end 138.8 73.5) (width 0.25) (layer "B.Cu") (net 1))
 (segment (start 104.63 139.75) (end 116.95 139.75) (width 0.6) (layer "B.Cu") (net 1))
 (segment (start 127.4395 74.5) (end 130.3875 77.448) (width 0.6) (layer "B.Cu") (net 1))
 (segment (start 137 75.3) (end 136 76.3) (width 0.25) (layer "B.Cu") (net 1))
 (segment (start 126.552 77.448) (end 122.2 81.8) (width 0.25) (layer "B.Cu") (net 1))
 (segment (start 72.126 90.326) (end 72.126 82.238) (width 0.6) (layer "B.Cu") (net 43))
 (segment (start 84.93 97.97) (end 79.77 97.97) (width 0.6) (layer "B.Cu") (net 43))
 (segment (start 79.77 97.97) (end 72.126 90.326) (width 0.6) (layer "B.Cu") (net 43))
 (segment (start 84.93 92.89) (end 78.778 92.89) (width 0.5) (layer "F.Cu") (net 11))
 (segment (start 78.778 92.89) (end 75.126 89.238) (width 0.5) (layer "F.Cu") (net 11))
 (segment (start 82.4125 125.3) (end 86.5 121.2125) (width 0.25) (layer "B.Cu") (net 11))
 (segment (start 86.5 94.46) (end 84.93 92.89) (width 0.25) (layer "B.Cu") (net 11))
 (segment (start 86.5 121.2125) (end 86.5 94.46) (width 0.25) (layer "B.Cu") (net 11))
 (segment (start 93.314 73.3) (end 96.1 76.086) (width 0.25) (layer "F.Cu") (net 10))
 (segment (start 96.1 76.086) (end 96.1 89.66) (width 0.25) (layer "F.Cu") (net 10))
 (segment (start 92.87 95.43) (end 92.87 92.89) (width 0.6) (layer "F.Cu") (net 10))
 (segment (start 96.1 89.66) (end 92.87 92.89) (width 0.25) (layer "F.Cu") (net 10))
 (segment (start 88.0125 100.2875) (end 92.87 95.43) (width 0.6) (layer "B.Cu") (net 10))
 (segment (start 88.0125 125.3) (end 88.0125 100.2875) (width 0.6) (layer "B.Cu") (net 10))
 (segment (start 83.054 83.508) (end 83.054 87.454) (width 0.6) (layer "F.Cu") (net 16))
 (segment (start 86.78 106.6) (end 75.1 106.6) (width 0.6) (layer "F.Cu") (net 16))
 (segment (start 88.4 92.8) (end 88.4 96.04) (width 0.6) (layer "F.Cu") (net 16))
 (segment (start 83.054 87.454) (end 88.4 92.8) (width 0.6) (layer "F.Cu") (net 16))
 (segment (start 92.87 100.51) (end 86.78 106.6) (width 0.6) (layer "F.Cu") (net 16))
 (segment (start 88.4 96.04) (end 92.87 100.51) (width 0.6) (layer "F.Cu") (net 16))
 (segment (start 113.44 138.4) (end 113.44 130.28) (width 0.25) (layer "F.Cu") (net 5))
 (segment (start 113.44 130.28) (end 117.34 126.38) (width 0.25) (layer "F.Cu") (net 5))
 (segment (start 102.3 77.7) (end 106.9 82.3) (width 0.6) (layer "F.Cu") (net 17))
 (segment (start 106.9 82.3) (end 106.9 86.02) (width 0.6) (layer "F.Cu") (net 17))
 (segment (start 106.9 86.02) (end 102.1 90.82) (width 0.6) (layer "F.Cu") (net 17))
 (via (at 102.3 77.7) (size 0.8) (drill 0.4) (layers "F.Cu" "B.Cu") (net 17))
 (segment (start 102.3 69.34) (end 102.3 77.7) (width 0.6) (layer "B.Cu") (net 17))
 (segment (start 95.96 63) (end 102.3 69.34) (width 0.6) (layer "B.Cu") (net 17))
 (segment (start 100.4 91.66) (end 102.1 93.36) (width 0.6) (layer "F.Cu") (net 18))
 (segment (start 100.4 79.1) (end 100.4 91.66) (width 0.6) (layer "F.Cu") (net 18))
 (via (at 100.4 79.1) (size 0.8) (drill 0.4) (layers "F.Cu" "B.Cu") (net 18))
 (segment (start 100.4 69.98) (end 100.4 79.1) (width 0.6) (layer "B.Cu") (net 18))
 (segment (start 93.42 63) (end 100.4 69.98) (width 0.6) (layer "B.Cu") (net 18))
 (segment (start 111.7 126.8) (end 115.98 131.08) (width 0.3) (layer "B.Cu") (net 6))
 (segment (start 115.98 131.08) (end 115.98 138.4) (width 0.3) (layer "B.Cu") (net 6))
 (segment (start 102.1 106.06) (end 111.7 115.66) (width 0.3) (layer "B.Cu") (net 6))
 (segment (start 111.7 115.66) (end 111.7 126.8) (width 0.3) (layer "B.Cu") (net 6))
 (segment (start 125.9025 94.87) (end 122.9 97.8725) (width 0.25) (layer "F.Cu") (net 13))
 (segment (start 122.9 97.8725) (end 122.9 104) (width 0.25) (layer "F.Cu") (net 13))
 (segment (start 136.62 105.5875) (end 136.62 109.6) (width 0.25) (layer "F.Cu") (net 13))
 (segment (start 117.44 108.5) (end 117.34 108.6) (width 0.25) (layer "F.Cu") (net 13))
 (segment (start 122.9 104) (end 118.4 108.5) (width 0.25) (layer "F.Cu") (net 13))
 (segment (start 125.9025 94.87) (end 136.62 105.5875) (width 0.25) (layer "F.Cu") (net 13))
 (segment (start 118.4 108.5) (end 117.44 108.5) (width 0.25) (layer "F.Cu") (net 13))
 (segment (start 121.1 102.3) (end 117.34 106.06) (width 0.25) (layer "F.Cu") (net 12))
 (segment (start 125.9025 92.33) (end 139.16 105.5875) (width 0.25) (layer "F.Cu") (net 12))
 (segment (start 139.16 105.5875) (end 139.16 109.6) (width 0.25) (layer "F.Cu") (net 12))
 (segment (start 125.9025 92.33) (end 121.1 97.1325) (width 0.25) (layer "F.Cu") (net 12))
 (segment (start 121.1 97.1325) (end 121.1 102.3) (width 0.25) (layer "F.Cu") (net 12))
 (segment (start 110.9 132.64) (end 102.1 123.84) (width 0.25) (layer "F.Cu") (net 4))
 (segment (start 110.9 132.64) (end 110.9 138.4) (width 0.25) (layer "F.Cu") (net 4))
 (segment (start 108.36 138.4) (end 108.36 132.64) (width 0.25) (layer "F.Cu") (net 3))
 (segment (start 108.36 132.64) (end 102.1 126.38) (width 0.25) (layer "F.Cu") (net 3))
 (segment (start 81.6 113.250121) (end 91.549879 113.250121) (width 0.6) (layer "F.Cu") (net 8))
 (segment (start 109.8 74.5) (end 109.8 85.8) (width 0.6) (layer "F.Cu") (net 8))
 (segment (start 109.8 85.8) (end 109.8 85.82) (width 0.6) (layer "F.Cu") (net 8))
 (segment (start 84.93 95.43) (end 83.865 96.495) (width 0.6) (layer "F.Cu") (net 8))
 (segment (start 83.865 96.495) (end 83.865 99.445) (width 0.6) (layer "F.Cu") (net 8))
 (segment (start 109.8 85.82) (end 117.34 93.36) (width 0.6) (layer "F.Cu") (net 8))
 (segment (start 83.865 99.445) (end 84.93 100.51) (width 0.6) (layer "F.Cu") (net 8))
 (segment (start 91.549879 113.250121) (end 91.6 113.2) (width 0.6) (layer "F.Cu") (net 8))
 (via (at 109.8 85.8) (size 0.8) (drill 0.4) (layers "F.Cu" "B.Cu") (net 8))
 (segment (start 83.896138 95.43) (end 84.93 95.43) (width 0.6) (layer "B.Cu") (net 8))
 (segment (start 93.214 83.508) (end 107.508 83.508) (width 0.6) (layer "B.Cu") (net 8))
 (segment (start 92.08263 83.508) (end 93.214 83.508) (width 0.6) (layer "B.Cu") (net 8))
 (segment (start 84.93 95.43) (end 83.865 94.365) (width 0.6) (layer "B.Cu") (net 8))
 (segment (start 84.93 109.920121) (end 84.93 100.51) (width 0.6) (layer "B.Cu") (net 8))
 (segment (start 83.865 91.72563) (end 92.08263 83.508) (width 0.6) (layer "B.Cu") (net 8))
 (segment (start 74.626 82.238) (end 74.626 86.159862) (width 0.6) (layer "B.Cu") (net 8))
 (segment (start 107.508 83.508) (end 109.8 85.8) (width 0.6) (layer "B.Cu") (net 8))
 (segment (start 81.6 113.250121) (end 84.93 109.920121) (width 0.6) (layer "B.Cu") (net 8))
 (segment (start 83.865 94.365) (end 83.865 91.72563) (width 0.6) (layer "B.Cu") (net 8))
 (segment (start 74.626 86.159862) (end 83.896138 95.43) (width 0.6) (layer "B.Cu") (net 8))
 (segment (start 77.8 116.3) (end 90.338478 116.3) (width 0.6) (layer "F.Cu") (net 7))
 (segment (start 75.126 99.398) (end 71.4 103.124) (width 0.6) (layer "F.Cu") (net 7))
 (segment (start 71.4 109.9) (end 75.1 113.6) (width 0.6) (layer "F.Cu") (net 7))
 (segment (start 71.4 103.124) (end 71.4 109.9) (width 0.6) (layer "F.Cu") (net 7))
 (segment (start 92.9 111) (end 91.6 109.7) (width 0.6) (layer "F.Cu") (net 7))
 (segment (start 90.338478 116.3) (end 92.9 113.738478) (width 0.6) (layer "F.Cu") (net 7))
 (segment (start 75.1 113.6) (end 77.8 116.3) (width 0.6) (layer "F.Cu") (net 7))
 (segment (start 92.9 113.738478) (end 92.9 111) (width 0.6) (layer "F.Cu") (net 7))
 (segment (start 99.042 102.258) (end 105.902 102.258) (width 0.6) (layer "B.Cu") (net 7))
 (segment (start 91.6 109.7) (end 99.042 102.258) (width 0.6) (layer "B.Cu") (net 7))
 (segment (start 105.902 102.258) (end 117.34 90.82) (width 0.6) (layer "B.Cu") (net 7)))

